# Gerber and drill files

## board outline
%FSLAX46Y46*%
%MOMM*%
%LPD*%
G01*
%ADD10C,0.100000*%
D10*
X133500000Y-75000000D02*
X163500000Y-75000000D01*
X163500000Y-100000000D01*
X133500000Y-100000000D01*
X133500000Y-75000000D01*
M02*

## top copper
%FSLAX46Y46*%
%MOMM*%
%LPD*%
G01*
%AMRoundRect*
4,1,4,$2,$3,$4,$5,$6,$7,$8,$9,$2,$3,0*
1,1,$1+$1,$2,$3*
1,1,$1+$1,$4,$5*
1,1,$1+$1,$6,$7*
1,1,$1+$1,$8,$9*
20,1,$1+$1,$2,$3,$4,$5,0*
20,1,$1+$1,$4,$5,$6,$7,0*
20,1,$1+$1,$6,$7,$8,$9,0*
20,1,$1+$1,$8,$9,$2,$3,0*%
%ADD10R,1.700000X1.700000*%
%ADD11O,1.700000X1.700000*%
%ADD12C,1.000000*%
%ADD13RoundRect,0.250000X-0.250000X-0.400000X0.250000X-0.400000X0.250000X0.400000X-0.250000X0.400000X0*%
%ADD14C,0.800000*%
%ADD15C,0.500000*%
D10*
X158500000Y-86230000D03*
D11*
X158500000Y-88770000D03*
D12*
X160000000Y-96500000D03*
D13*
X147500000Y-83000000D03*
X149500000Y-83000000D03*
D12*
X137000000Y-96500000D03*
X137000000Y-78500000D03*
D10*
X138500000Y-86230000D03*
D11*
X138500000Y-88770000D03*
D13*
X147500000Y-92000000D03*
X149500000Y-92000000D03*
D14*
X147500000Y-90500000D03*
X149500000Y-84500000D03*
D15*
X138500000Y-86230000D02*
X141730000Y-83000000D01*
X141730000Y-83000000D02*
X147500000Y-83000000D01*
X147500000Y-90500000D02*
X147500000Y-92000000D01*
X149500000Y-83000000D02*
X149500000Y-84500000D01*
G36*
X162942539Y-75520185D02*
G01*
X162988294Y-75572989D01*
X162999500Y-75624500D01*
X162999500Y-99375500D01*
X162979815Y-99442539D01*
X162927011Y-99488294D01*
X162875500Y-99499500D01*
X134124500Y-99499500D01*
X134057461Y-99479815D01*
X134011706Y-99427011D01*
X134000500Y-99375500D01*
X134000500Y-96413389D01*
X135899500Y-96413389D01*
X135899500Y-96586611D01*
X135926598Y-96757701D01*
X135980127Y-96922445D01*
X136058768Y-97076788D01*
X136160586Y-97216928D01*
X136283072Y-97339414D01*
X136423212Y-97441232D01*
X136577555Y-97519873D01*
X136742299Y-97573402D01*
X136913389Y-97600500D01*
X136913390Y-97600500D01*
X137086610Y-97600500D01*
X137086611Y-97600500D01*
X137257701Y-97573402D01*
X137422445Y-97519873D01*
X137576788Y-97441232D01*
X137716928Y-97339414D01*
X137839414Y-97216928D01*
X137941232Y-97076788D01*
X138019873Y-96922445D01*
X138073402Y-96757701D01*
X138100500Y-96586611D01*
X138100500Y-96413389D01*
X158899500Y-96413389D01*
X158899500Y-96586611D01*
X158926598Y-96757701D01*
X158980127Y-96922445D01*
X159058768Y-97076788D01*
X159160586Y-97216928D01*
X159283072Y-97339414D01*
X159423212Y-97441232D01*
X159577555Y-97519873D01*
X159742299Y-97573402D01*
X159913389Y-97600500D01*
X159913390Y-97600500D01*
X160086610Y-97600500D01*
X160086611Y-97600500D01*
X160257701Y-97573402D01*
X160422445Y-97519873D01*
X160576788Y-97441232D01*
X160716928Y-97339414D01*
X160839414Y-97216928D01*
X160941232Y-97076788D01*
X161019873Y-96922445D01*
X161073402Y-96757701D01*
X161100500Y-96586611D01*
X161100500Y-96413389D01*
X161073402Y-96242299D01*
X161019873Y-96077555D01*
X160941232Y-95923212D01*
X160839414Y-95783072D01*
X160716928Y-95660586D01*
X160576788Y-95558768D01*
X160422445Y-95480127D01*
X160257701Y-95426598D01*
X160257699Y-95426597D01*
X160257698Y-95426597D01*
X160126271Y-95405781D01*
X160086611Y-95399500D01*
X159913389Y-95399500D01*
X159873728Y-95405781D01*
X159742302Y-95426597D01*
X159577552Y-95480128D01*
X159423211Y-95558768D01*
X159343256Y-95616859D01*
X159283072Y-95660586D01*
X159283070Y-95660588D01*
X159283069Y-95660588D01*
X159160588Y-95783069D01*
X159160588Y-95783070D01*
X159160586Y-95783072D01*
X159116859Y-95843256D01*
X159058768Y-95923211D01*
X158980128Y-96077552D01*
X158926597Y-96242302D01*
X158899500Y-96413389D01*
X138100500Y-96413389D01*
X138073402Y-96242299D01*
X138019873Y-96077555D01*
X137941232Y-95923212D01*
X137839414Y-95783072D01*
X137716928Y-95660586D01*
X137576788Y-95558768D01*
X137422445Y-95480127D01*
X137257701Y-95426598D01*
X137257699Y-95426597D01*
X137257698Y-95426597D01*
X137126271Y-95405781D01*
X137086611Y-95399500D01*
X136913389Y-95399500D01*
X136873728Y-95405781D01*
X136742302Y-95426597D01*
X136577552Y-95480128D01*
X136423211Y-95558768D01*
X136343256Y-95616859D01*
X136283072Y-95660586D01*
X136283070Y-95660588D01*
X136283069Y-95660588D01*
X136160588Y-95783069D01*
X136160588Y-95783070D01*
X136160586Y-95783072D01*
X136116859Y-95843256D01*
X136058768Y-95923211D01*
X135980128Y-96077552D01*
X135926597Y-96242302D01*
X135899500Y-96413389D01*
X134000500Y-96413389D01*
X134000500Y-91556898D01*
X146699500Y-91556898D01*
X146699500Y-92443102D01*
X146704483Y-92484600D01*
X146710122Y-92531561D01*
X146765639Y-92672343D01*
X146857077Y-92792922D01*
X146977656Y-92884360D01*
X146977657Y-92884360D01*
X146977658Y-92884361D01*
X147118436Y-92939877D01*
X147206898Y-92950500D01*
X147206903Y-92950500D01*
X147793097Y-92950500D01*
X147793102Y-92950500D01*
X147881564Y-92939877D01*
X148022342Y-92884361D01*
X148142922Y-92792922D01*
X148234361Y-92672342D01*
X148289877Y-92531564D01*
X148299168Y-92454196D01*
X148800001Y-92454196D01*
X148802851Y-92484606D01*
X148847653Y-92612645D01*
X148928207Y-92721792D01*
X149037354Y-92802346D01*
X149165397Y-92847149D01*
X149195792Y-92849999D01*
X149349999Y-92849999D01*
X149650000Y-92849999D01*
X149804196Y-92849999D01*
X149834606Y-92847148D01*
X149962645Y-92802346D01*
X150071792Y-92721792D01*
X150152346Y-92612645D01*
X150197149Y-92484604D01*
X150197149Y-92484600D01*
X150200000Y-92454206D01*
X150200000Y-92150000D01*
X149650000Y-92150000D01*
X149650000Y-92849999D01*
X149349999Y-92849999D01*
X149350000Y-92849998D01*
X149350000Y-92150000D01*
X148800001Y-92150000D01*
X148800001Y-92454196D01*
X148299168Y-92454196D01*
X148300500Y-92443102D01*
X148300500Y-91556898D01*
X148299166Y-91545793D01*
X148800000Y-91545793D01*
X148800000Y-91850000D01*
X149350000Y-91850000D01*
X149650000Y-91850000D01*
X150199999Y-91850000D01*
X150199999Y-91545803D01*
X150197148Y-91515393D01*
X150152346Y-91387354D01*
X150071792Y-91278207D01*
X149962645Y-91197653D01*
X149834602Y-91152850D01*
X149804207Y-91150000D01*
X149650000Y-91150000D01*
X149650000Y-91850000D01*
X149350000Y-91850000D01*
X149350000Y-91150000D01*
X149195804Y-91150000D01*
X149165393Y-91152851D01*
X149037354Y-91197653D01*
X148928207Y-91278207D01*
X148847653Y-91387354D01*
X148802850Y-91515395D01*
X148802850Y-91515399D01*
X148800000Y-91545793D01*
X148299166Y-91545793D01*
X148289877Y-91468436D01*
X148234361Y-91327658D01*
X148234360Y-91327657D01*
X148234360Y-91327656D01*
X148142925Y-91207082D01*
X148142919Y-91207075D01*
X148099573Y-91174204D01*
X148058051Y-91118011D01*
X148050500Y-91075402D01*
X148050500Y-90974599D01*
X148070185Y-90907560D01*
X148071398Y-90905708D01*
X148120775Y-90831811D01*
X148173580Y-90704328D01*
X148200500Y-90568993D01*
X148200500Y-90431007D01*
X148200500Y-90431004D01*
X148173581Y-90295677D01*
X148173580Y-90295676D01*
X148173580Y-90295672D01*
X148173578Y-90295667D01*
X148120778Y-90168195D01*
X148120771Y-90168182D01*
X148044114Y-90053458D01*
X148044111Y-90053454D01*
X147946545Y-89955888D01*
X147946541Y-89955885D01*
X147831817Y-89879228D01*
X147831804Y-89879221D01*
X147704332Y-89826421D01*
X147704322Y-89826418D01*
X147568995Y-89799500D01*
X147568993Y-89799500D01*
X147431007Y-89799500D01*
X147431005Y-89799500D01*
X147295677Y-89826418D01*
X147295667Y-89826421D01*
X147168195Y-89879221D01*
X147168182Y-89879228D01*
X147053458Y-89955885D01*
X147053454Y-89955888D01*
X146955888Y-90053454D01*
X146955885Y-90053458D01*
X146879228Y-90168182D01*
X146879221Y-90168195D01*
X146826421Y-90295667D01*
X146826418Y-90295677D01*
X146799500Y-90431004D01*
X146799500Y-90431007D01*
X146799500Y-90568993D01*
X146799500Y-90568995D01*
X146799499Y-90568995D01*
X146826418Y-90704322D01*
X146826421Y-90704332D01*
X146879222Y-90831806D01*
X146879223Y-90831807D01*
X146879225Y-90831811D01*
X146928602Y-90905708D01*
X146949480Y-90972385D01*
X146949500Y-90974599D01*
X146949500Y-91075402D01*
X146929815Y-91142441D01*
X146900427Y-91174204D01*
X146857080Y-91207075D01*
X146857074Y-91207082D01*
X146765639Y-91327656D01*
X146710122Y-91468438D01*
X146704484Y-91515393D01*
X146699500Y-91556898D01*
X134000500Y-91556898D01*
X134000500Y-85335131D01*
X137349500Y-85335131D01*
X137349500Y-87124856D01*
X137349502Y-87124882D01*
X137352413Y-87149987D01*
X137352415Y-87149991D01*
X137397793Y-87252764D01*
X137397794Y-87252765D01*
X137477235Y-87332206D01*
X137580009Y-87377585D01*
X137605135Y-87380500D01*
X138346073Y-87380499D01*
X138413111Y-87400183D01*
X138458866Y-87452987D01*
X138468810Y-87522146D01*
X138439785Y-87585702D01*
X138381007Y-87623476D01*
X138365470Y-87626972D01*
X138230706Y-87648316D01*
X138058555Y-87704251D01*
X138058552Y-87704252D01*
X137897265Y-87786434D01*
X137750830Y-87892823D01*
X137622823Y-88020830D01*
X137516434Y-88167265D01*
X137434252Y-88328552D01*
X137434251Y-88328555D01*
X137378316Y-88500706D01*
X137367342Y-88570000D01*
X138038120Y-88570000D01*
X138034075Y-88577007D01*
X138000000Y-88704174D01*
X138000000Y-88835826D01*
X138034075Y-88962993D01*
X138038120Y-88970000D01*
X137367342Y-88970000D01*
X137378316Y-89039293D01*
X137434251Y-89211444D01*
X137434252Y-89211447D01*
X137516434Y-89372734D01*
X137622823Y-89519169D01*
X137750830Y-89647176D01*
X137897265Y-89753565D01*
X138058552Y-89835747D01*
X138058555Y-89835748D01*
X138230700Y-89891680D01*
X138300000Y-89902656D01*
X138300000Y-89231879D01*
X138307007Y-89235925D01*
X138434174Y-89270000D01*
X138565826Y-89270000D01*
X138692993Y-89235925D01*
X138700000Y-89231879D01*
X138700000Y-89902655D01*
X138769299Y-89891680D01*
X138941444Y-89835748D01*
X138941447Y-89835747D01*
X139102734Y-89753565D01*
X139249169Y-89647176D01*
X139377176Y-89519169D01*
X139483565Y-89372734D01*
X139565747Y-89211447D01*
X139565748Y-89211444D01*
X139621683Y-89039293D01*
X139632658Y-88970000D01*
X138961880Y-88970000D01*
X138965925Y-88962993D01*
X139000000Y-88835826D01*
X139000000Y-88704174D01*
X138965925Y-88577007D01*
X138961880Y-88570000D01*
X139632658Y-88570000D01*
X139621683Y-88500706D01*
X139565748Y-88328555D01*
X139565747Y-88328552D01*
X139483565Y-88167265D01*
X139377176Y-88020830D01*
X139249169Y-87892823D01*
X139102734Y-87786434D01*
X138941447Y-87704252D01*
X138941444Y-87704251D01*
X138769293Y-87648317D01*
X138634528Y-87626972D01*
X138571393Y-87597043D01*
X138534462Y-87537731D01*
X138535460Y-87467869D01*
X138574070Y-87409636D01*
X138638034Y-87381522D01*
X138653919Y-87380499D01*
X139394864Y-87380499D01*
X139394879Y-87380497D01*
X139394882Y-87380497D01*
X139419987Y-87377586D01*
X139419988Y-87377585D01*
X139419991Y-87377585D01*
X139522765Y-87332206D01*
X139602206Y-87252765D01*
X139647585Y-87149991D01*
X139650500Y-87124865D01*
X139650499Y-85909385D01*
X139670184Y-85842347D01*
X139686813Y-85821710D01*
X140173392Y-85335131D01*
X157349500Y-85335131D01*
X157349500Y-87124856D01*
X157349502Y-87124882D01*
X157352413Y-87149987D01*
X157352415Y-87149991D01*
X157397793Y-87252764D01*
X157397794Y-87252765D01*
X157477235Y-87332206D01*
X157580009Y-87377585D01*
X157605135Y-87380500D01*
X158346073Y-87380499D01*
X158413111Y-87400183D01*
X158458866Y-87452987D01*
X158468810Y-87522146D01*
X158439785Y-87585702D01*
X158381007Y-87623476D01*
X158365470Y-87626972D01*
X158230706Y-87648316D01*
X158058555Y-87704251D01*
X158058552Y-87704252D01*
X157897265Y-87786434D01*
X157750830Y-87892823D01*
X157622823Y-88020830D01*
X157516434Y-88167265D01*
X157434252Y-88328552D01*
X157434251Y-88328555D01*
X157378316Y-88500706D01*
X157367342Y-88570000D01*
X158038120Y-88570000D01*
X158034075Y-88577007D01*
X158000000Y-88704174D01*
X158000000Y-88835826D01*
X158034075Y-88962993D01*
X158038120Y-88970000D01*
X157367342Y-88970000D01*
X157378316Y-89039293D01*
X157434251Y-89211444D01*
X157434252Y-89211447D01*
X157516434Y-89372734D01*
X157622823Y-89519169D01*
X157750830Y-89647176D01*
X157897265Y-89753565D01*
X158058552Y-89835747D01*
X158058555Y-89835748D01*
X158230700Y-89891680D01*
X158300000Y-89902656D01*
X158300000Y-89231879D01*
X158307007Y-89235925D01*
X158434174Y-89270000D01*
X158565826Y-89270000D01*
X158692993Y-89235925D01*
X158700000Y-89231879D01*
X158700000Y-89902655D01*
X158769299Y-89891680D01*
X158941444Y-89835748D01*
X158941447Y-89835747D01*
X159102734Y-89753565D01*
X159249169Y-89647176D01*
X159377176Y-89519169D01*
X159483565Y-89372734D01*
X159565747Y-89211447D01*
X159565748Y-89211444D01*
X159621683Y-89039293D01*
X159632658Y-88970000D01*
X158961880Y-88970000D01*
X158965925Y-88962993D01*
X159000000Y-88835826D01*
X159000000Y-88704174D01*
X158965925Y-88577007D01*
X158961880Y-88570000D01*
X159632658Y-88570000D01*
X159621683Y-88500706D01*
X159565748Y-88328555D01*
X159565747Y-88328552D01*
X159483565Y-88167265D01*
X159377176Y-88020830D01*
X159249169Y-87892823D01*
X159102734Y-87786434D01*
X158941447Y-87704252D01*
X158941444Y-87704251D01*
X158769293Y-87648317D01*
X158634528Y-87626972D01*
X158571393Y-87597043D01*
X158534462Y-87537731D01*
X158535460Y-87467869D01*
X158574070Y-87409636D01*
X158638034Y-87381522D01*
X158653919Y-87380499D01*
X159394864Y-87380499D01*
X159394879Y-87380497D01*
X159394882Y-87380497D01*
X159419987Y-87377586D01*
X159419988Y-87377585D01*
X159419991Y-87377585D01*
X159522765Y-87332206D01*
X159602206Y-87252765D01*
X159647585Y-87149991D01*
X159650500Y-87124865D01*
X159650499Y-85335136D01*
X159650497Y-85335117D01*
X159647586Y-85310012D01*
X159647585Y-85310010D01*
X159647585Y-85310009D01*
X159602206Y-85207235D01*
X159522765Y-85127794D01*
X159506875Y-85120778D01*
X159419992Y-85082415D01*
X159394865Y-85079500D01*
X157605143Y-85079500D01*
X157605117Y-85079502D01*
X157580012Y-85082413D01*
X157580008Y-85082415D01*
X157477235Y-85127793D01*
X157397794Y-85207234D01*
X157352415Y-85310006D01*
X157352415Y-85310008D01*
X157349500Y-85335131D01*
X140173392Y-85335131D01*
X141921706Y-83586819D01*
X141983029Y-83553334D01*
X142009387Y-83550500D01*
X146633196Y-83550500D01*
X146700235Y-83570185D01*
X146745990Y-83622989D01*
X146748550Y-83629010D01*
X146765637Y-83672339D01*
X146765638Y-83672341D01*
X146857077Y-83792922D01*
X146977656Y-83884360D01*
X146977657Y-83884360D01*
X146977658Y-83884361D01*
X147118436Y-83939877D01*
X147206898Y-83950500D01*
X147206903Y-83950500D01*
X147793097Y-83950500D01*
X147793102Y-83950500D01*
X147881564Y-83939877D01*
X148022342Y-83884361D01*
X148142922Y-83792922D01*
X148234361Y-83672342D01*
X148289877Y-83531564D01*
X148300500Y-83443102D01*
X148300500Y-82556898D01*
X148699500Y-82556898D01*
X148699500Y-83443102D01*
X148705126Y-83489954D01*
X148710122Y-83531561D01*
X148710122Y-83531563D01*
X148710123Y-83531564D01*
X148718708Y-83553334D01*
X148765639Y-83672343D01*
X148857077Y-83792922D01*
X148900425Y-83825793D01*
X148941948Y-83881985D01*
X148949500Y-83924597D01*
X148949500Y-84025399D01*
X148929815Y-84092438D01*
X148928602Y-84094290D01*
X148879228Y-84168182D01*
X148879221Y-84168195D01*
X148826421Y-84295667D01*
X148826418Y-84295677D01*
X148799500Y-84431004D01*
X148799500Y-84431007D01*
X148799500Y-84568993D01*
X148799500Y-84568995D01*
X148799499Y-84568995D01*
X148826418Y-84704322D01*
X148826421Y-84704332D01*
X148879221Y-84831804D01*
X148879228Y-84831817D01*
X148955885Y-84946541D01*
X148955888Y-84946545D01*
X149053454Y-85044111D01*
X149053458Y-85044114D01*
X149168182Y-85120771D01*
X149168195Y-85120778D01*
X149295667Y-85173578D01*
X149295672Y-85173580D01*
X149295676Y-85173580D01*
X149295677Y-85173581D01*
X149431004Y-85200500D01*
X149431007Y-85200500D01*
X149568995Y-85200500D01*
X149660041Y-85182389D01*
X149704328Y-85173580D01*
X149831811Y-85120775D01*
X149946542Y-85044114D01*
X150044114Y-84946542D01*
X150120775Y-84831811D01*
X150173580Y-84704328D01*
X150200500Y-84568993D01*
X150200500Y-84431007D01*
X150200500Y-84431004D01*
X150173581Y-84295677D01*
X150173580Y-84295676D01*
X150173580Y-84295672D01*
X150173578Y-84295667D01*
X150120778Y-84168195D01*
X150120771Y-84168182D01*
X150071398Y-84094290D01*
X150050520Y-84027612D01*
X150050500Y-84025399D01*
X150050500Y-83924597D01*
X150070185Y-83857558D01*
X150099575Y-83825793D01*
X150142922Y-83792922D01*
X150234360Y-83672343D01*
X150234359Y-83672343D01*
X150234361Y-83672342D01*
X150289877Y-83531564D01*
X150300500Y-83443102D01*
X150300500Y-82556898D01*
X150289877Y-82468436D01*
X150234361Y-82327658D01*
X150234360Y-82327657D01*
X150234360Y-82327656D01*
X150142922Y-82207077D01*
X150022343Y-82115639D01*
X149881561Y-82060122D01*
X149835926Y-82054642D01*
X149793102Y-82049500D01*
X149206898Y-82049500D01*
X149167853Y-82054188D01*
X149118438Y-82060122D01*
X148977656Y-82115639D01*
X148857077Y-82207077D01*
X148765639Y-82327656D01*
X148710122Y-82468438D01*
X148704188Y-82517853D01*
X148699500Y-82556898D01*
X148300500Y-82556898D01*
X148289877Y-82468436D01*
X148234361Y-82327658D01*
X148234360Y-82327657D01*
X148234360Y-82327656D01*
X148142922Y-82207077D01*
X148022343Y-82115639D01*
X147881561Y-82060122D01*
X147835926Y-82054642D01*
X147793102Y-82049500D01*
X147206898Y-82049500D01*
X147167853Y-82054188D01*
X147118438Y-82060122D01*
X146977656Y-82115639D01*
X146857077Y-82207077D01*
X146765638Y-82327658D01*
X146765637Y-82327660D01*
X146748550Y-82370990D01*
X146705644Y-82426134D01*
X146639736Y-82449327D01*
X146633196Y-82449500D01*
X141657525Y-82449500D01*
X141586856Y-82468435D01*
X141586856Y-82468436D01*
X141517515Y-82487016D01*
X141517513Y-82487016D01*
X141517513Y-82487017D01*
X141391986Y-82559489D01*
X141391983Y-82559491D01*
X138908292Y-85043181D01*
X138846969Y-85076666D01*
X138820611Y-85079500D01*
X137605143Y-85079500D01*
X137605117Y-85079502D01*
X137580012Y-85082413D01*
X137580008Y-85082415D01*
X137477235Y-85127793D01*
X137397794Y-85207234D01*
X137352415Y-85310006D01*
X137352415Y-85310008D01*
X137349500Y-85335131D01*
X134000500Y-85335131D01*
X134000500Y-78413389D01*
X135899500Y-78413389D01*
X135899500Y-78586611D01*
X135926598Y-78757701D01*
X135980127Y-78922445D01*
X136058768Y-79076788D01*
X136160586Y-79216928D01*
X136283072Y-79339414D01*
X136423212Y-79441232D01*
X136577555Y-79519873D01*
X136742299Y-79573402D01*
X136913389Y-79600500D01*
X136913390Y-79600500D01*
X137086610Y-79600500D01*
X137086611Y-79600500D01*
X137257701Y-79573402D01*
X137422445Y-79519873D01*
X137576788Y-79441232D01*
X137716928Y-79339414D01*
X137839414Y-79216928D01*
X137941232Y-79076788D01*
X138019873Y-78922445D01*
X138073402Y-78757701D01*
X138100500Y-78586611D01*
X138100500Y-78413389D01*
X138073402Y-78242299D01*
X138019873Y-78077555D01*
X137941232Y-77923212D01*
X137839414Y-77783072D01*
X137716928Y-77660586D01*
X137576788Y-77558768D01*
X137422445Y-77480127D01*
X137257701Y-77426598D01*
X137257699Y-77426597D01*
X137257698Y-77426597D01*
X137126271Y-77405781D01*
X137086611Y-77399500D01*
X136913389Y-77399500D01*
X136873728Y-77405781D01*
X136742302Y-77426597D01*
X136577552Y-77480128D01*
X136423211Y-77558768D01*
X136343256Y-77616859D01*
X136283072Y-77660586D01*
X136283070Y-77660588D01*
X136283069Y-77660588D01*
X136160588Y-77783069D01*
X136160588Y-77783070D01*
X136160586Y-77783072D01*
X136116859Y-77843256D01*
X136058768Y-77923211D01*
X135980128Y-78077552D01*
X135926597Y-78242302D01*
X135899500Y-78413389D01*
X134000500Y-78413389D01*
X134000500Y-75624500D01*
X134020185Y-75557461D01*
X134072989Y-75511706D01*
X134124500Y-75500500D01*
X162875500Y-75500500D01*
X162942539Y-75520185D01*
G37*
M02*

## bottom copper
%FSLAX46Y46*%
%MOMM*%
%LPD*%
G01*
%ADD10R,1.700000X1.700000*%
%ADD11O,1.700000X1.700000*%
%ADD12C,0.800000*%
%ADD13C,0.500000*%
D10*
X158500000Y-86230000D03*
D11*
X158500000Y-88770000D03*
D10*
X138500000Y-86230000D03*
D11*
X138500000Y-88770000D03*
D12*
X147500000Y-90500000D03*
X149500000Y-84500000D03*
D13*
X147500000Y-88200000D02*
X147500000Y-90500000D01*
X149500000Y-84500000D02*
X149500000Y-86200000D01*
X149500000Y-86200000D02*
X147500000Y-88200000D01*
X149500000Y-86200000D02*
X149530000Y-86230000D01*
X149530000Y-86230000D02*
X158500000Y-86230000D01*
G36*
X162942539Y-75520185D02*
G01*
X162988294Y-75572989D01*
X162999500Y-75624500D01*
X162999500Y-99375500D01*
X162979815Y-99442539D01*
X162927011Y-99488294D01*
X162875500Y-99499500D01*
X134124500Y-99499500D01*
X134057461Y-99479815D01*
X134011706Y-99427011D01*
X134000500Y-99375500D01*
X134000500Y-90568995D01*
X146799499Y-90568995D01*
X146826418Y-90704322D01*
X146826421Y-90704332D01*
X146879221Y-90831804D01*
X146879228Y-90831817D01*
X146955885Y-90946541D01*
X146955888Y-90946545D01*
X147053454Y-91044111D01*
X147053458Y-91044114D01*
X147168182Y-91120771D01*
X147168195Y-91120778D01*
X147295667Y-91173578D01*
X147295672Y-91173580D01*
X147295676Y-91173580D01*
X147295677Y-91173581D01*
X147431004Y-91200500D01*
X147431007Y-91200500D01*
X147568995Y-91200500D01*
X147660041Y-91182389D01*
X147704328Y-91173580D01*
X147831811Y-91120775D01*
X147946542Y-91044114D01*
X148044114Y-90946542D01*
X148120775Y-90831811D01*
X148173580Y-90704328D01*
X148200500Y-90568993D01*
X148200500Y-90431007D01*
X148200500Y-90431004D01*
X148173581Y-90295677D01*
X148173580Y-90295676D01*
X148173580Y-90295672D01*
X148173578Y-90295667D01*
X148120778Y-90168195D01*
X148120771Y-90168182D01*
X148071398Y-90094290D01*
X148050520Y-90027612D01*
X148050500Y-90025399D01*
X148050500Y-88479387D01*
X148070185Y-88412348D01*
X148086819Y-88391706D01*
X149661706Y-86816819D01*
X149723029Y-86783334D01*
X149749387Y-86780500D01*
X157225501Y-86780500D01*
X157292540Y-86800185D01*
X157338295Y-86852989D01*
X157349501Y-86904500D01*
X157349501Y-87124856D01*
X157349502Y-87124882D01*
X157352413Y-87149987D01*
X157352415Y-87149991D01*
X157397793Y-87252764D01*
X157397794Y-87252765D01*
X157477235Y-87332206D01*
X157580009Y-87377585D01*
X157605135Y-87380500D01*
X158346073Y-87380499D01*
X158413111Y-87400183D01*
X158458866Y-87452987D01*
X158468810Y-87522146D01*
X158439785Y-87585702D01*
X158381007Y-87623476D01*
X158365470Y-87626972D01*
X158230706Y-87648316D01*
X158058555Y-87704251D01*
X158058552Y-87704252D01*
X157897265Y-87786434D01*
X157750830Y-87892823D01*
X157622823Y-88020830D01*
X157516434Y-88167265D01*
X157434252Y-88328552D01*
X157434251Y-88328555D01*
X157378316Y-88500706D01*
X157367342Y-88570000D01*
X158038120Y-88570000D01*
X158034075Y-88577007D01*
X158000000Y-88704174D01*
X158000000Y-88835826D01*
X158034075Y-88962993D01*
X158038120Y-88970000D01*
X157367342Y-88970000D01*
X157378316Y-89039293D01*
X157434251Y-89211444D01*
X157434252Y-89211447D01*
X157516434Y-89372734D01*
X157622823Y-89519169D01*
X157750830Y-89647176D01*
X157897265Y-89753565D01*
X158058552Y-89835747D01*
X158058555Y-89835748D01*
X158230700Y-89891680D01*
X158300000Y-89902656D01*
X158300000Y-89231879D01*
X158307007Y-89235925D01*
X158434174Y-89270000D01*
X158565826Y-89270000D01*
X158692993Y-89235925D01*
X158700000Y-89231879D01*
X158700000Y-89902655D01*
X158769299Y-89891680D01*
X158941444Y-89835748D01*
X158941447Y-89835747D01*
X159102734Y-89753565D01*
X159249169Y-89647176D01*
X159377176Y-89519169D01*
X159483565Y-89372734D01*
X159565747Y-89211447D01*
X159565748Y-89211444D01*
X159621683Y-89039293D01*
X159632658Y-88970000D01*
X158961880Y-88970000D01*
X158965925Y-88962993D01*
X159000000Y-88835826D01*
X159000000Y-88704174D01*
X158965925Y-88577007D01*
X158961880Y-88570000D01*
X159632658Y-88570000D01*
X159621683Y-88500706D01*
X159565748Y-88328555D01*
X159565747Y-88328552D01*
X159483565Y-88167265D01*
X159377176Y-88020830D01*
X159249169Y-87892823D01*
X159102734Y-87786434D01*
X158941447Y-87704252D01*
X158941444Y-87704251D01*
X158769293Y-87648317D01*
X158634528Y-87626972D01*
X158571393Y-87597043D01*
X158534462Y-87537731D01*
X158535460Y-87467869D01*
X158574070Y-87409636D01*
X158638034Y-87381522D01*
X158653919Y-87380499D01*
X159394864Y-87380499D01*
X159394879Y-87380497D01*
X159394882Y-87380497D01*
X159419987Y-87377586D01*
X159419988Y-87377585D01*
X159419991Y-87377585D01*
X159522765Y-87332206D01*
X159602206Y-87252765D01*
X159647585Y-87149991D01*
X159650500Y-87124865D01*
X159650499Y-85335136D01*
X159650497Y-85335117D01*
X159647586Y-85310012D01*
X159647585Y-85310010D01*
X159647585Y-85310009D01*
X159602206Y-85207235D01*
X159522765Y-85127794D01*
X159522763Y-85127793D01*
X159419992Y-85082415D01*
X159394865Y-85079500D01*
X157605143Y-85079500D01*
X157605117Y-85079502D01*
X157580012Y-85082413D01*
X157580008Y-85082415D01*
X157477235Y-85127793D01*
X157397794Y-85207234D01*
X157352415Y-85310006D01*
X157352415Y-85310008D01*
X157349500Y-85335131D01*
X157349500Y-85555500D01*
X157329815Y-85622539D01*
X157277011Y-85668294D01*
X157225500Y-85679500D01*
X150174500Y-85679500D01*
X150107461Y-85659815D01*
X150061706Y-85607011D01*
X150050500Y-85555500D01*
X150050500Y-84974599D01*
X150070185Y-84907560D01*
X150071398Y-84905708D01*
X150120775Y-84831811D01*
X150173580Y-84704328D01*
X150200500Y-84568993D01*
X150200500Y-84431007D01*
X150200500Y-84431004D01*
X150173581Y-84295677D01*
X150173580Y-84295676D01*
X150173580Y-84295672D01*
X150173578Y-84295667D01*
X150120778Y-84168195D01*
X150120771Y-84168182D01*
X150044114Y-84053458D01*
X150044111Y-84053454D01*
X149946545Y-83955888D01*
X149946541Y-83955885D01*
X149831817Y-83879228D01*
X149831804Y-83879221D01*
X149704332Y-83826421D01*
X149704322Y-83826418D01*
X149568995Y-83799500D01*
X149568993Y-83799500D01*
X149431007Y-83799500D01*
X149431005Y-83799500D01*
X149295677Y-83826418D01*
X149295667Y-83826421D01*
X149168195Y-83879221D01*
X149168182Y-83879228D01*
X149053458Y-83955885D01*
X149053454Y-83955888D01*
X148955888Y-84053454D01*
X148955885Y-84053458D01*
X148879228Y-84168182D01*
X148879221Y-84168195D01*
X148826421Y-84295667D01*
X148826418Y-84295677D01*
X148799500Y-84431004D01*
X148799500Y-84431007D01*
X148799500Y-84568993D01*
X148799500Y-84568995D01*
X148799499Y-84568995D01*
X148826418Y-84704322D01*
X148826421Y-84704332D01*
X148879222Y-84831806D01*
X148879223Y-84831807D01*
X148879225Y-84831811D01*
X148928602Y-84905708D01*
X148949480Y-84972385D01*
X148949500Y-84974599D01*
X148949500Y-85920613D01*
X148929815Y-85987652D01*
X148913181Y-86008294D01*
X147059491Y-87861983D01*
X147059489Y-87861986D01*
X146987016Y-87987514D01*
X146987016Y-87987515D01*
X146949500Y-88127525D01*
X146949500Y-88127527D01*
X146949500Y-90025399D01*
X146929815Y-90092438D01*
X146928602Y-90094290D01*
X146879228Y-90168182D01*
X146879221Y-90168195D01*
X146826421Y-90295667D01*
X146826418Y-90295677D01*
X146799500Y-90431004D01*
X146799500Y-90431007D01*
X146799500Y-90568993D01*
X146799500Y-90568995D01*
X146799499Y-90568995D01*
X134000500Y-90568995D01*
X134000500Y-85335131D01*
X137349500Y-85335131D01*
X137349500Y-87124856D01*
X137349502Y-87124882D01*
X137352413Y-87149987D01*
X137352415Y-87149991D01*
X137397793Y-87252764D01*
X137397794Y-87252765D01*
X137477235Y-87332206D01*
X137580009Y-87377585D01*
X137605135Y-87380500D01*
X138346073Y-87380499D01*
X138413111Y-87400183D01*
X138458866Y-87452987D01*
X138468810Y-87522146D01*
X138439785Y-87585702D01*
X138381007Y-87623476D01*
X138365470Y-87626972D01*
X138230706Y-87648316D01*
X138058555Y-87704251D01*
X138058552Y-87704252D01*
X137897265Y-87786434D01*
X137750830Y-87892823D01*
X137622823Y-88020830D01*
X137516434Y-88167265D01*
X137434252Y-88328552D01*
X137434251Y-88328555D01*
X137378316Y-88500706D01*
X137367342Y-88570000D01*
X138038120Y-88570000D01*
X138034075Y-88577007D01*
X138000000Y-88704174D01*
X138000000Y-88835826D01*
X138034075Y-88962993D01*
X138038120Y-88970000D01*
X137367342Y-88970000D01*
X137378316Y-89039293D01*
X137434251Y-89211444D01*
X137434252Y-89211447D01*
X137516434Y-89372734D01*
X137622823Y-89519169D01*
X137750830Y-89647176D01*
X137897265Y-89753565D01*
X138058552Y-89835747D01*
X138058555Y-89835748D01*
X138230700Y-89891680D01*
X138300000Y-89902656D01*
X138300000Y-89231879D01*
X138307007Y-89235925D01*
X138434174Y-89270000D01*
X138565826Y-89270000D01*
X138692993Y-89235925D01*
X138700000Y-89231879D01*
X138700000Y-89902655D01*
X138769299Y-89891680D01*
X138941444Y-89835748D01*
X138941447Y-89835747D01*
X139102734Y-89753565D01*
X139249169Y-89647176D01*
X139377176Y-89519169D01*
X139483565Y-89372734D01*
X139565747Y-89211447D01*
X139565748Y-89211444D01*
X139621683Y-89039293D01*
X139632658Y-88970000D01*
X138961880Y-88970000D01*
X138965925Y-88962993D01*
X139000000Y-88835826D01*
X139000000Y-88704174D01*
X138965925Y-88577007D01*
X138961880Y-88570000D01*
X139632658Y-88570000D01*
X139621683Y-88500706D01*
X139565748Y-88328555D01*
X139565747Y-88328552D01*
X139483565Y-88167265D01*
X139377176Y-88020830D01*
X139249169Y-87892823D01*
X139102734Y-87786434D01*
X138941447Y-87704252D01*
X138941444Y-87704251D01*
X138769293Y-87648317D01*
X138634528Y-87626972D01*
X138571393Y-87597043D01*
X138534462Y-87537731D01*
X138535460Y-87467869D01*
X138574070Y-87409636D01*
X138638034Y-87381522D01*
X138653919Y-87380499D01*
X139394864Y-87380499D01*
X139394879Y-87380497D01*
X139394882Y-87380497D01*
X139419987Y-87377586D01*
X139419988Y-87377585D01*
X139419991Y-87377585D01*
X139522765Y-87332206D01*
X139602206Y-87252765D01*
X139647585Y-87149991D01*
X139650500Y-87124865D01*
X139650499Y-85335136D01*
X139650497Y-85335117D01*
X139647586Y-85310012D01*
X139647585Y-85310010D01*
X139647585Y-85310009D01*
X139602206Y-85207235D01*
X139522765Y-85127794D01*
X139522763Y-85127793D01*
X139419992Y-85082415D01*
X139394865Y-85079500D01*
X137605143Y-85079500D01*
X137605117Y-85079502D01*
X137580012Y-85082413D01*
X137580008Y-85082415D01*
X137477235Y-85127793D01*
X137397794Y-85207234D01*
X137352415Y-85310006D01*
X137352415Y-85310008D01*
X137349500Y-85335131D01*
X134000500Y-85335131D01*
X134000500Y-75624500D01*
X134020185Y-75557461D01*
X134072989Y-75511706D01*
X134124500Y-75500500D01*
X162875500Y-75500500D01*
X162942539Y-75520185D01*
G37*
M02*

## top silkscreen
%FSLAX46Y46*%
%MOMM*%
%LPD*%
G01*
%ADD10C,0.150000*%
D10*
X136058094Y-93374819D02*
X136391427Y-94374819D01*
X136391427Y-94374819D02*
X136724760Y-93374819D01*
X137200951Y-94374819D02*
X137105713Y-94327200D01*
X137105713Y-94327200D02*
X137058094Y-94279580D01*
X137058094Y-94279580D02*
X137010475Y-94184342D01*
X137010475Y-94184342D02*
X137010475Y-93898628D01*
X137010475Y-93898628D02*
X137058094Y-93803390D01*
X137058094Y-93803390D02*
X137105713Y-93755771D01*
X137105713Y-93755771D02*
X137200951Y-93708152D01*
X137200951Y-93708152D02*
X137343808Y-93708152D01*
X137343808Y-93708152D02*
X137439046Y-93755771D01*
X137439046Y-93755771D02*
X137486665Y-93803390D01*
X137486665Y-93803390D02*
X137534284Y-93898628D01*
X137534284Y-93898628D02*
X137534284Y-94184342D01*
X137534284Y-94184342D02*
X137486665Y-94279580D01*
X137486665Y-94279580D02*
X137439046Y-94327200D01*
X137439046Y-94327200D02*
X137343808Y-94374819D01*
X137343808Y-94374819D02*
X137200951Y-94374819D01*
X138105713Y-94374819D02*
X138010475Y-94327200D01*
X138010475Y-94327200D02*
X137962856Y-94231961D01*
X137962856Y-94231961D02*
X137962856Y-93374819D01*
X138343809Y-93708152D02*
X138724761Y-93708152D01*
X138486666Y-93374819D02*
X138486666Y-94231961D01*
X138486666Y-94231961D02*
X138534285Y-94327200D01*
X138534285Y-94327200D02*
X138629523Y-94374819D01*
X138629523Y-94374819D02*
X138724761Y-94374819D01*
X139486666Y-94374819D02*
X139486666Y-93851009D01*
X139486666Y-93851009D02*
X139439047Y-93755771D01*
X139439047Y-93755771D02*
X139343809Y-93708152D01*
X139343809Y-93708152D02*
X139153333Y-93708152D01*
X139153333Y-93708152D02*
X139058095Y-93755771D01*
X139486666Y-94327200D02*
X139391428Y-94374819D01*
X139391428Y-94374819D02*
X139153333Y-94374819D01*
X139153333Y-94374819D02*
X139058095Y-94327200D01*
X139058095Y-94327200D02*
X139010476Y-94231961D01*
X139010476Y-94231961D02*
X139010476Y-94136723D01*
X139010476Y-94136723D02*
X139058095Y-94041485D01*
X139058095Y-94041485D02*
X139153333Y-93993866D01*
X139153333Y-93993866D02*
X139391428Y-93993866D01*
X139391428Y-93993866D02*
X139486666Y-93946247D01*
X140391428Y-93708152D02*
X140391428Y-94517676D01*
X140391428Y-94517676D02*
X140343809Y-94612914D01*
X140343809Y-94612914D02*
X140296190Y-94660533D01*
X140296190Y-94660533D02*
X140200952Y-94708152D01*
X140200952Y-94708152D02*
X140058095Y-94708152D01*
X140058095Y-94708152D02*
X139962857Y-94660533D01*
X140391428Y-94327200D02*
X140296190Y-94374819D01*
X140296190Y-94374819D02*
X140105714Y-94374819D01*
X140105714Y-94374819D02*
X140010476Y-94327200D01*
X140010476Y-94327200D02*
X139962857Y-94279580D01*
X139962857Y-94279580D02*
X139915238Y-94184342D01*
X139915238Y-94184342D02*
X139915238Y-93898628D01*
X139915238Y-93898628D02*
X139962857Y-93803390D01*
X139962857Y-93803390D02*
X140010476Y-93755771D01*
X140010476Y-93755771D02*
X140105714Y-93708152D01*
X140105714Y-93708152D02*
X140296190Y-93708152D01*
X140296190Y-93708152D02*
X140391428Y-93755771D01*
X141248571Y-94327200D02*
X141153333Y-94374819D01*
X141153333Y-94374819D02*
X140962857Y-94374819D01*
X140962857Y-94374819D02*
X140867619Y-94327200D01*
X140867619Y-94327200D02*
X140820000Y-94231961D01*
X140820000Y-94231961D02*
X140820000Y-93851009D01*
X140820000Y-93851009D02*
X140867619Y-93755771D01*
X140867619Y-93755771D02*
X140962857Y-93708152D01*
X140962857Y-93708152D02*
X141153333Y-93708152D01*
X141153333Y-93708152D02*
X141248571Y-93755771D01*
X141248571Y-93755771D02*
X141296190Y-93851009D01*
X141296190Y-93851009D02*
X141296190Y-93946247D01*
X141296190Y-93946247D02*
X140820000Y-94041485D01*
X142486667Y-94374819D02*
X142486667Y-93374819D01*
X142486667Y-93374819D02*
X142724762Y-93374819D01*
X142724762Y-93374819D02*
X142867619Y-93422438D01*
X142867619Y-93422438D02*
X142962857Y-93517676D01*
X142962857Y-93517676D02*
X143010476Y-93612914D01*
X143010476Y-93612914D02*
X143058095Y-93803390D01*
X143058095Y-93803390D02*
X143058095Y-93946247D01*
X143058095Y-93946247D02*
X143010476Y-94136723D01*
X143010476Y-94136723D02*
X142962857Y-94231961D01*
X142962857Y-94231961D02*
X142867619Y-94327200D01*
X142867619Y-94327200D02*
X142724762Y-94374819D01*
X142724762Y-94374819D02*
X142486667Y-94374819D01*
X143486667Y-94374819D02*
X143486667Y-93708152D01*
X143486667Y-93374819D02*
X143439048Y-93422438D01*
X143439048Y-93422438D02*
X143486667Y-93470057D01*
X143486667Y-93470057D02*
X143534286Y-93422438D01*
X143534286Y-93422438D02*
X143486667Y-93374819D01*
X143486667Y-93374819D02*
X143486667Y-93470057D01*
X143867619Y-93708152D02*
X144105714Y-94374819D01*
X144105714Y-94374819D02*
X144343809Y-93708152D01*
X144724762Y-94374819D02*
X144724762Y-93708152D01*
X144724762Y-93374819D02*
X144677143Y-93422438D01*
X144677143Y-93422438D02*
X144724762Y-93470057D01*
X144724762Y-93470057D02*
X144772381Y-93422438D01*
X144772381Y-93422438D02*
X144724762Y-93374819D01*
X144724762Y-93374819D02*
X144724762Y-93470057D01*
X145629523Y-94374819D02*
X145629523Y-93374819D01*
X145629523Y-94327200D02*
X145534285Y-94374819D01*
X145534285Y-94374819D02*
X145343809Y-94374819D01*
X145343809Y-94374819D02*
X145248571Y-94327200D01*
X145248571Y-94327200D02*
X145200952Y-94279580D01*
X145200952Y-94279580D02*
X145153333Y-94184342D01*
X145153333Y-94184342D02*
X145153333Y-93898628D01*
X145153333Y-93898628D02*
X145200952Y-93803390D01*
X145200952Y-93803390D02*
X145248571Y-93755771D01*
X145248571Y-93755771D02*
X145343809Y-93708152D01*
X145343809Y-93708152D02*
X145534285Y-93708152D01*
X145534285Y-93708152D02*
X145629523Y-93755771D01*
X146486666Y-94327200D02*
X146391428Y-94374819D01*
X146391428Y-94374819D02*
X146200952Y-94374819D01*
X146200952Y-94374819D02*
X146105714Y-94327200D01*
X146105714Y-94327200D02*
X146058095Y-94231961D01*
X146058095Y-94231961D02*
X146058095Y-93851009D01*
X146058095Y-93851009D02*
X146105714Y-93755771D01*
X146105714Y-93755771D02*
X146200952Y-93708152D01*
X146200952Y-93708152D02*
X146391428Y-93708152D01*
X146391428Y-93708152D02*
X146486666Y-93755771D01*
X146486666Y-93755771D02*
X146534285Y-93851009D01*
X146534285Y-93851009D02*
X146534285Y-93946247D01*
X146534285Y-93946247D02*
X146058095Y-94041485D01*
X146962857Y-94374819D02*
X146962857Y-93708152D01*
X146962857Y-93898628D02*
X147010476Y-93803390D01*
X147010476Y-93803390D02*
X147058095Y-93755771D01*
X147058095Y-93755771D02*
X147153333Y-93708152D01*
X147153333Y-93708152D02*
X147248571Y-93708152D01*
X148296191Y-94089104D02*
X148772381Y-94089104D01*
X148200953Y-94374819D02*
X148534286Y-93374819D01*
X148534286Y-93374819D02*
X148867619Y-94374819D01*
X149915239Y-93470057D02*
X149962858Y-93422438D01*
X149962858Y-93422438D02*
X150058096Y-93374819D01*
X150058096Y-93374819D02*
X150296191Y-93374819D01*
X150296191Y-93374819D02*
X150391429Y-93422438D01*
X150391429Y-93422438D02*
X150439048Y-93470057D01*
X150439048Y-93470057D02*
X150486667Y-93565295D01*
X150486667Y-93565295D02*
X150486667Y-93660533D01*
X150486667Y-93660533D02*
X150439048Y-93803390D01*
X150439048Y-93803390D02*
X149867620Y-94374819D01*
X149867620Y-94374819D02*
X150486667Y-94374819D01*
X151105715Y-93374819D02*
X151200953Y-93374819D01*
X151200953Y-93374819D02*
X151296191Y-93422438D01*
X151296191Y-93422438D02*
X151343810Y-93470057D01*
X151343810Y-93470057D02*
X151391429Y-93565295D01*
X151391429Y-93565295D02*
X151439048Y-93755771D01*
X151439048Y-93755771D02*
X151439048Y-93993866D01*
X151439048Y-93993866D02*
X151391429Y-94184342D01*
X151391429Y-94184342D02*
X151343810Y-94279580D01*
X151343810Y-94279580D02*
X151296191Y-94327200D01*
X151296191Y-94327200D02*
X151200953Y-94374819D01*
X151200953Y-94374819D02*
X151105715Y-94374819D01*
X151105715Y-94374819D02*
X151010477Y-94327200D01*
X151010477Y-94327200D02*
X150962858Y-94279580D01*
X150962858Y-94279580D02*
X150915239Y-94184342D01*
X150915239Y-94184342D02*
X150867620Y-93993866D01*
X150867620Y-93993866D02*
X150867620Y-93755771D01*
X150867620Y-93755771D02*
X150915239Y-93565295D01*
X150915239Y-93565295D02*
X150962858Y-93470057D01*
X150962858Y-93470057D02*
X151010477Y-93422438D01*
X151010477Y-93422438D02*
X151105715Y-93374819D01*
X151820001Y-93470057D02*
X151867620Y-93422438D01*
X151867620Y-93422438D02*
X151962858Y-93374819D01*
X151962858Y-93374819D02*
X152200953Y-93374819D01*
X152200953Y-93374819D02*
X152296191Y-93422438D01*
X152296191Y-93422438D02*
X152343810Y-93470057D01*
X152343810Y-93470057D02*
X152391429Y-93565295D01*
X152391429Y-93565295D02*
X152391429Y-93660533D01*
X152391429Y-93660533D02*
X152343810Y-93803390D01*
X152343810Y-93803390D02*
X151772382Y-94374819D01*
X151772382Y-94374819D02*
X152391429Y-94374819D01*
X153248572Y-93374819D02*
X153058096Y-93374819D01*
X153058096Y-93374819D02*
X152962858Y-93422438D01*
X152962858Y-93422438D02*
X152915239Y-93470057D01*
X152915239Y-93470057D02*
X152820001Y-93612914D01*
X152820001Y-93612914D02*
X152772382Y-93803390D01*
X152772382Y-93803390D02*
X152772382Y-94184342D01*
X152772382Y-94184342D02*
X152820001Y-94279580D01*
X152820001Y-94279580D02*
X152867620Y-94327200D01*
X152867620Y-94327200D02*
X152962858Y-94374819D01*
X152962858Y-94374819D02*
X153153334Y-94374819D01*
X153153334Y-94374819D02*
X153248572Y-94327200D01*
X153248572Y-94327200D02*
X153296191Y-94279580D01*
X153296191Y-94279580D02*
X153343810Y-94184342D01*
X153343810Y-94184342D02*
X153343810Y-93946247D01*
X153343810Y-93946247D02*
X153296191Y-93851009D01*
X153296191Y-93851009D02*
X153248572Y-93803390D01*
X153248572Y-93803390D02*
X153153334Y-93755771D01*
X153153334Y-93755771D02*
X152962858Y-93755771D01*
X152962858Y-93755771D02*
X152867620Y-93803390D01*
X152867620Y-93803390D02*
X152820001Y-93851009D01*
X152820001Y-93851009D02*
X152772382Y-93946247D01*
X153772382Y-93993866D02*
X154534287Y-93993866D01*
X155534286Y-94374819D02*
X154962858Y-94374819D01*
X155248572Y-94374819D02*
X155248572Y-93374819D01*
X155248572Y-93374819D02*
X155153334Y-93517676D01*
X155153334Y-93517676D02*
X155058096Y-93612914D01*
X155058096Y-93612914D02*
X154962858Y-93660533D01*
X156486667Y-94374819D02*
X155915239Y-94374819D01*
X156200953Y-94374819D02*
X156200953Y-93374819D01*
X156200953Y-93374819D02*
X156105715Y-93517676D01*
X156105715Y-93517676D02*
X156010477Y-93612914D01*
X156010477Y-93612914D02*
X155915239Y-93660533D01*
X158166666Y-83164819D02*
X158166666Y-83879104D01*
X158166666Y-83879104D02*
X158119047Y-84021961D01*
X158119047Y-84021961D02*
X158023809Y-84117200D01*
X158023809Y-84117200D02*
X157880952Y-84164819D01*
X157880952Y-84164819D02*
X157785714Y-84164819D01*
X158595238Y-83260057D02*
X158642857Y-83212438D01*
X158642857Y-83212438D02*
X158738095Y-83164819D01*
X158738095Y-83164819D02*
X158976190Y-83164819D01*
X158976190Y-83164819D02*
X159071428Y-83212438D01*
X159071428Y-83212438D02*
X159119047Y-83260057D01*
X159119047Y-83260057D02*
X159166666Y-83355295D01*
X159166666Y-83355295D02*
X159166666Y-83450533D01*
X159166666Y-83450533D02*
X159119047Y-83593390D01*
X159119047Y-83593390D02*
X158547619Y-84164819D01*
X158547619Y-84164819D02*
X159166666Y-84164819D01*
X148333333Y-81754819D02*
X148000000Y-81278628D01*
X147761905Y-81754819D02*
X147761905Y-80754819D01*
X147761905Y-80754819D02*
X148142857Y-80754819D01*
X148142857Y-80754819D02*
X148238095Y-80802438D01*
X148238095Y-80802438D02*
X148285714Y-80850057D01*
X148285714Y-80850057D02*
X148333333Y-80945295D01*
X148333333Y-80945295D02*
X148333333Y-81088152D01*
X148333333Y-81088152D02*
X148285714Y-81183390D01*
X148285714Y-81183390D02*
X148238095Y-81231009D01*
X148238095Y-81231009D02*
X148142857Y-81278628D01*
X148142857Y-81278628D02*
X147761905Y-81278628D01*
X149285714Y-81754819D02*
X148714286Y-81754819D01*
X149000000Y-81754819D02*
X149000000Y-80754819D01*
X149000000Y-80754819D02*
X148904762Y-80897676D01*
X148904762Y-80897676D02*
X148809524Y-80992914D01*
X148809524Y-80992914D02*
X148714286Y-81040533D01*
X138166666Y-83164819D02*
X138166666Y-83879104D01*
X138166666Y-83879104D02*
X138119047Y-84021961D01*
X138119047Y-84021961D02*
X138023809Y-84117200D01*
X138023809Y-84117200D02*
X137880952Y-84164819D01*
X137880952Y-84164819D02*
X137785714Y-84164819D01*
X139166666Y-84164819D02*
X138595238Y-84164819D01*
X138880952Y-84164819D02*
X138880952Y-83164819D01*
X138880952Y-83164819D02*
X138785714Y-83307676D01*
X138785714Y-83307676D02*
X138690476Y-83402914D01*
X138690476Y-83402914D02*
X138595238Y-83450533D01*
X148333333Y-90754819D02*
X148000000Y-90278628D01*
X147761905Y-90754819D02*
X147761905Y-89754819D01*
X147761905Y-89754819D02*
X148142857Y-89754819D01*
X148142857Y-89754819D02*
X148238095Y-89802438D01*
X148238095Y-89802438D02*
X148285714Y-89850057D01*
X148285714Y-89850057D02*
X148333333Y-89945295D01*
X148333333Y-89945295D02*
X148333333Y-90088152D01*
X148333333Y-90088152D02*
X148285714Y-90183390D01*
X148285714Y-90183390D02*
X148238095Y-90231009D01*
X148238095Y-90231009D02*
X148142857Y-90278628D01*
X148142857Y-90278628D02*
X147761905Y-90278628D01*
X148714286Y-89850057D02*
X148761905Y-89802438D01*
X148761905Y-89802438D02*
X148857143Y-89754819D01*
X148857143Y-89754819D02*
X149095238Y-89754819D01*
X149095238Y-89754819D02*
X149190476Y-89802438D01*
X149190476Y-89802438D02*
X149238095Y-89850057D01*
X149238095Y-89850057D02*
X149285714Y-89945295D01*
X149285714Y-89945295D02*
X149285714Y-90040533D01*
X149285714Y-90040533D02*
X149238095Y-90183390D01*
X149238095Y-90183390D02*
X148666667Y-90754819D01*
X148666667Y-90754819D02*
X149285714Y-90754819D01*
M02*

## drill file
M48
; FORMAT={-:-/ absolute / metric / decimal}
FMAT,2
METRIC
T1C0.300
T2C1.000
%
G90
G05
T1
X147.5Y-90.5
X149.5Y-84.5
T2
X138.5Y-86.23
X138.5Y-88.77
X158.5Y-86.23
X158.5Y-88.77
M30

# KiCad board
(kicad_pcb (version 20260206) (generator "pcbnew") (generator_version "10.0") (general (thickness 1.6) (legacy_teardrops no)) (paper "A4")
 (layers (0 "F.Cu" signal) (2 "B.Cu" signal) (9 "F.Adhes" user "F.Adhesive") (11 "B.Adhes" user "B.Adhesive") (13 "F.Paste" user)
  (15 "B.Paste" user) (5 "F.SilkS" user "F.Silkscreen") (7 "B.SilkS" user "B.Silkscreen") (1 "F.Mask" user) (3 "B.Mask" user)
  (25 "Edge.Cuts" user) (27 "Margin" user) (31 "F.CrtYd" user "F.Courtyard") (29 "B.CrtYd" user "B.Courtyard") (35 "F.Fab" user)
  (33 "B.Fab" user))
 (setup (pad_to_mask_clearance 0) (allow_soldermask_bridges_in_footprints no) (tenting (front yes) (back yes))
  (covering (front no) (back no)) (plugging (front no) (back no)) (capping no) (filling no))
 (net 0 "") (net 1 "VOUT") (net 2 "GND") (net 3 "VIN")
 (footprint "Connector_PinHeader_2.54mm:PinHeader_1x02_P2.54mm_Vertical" (layer "F.Cu") (at 158.5 87.5)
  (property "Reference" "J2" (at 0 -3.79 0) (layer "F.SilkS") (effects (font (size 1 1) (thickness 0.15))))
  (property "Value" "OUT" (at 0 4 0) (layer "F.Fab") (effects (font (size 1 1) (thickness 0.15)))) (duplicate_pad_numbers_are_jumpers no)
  (pad "1" thru_hole rect (at 0 -1.27) (size 1.7 1.7) (drill 1) (layers "*.Cu" "*.Mask") (remove_unused_layers no) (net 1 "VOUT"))
  (pad "2" thru_hole oval (at 0 1.27) (size 1.7 1.7) (drill 1) (layers "*.Cu" "*.Mask") (remove_unused_layers no) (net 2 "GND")))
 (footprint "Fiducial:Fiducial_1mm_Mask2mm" (layer "F.Cu") (at 160 96.5)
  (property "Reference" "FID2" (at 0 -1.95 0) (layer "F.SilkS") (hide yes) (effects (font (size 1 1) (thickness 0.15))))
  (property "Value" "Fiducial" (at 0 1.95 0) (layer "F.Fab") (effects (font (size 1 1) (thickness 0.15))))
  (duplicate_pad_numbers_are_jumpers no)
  (pad "" smd circle (at 0 0) (size 1 1) (layers "F.Cu" "F.Mask") (solder_mask_margin 0.5) (clearance 0.6)))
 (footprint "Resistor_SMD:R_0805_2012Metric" (layer "F.Cu") (at 148.5 83)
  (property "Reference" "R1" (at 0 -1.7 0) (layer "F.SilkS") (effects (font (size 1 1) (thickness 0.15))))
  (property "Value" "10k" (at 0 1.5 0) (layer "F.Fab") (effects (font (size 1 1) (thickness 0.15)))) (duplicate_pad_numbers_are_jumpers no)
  (pad "1" smd roundrect (at -1 0) (size 1 1.3) (layers "F.Cu" "F.Mask" "F.Paste") (roundrect_rratio 0.25) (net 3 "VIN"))
  (pad "2" smd roundrect (at 1 0) (size 1 1.3) (layers "F.Cu" "F.Mask" "F.Paste") (roundrect_rratio 0.25) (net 1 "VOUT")))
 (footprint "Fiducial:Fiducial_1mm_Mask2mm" (layer "F.Cu") (at 137 96.5)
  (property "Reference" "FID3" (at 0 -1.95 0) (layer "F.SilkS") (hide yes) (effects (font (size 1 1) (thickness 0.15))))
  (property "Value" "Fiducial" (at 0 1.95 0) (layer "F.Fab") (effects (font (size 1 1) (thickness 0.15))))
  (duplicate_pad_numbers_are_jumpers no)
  (pad "" smd circle (at 0 0) (size 1 1) (layers "F.Cu" "F.Mask") (solder_mask_margin 0.5) (clearance 0.6)))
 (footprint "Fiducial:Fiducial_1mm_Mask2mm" (layer "F.Cu") (at 137 78.5)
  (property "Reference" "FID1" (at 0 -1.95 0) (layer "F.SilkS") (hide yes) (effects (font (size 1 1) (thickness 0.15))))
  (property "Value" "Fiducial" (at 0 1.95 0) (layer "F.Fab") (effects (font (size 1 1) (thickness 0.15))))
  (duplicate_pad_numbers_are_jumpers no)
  (pad "" smd circle (at 0 0) (size 1 1) (layers "F.Cu" "F.Mask") (solder_mask_margin 0.5) (clearance 0.6)))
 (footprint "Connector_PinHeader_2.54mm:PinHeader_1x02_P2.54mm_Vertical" (layer "F.Cu") (at 138.5 87.5)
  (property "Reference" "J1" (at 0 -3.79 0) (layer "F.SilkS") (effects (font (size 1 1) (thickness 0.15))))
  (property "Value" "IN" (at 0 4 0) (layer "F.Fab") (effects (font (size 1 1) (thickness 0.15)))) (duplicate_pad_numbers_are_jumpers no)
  (pad "1" thru_hole rect (at 0 -1.27) (size 1.7 1.7) (drill 1) (layers "*.Cu" "*.Mask") (remove_unused_layers no) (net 3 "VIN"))
  (pad "2" thru_hole oval (at 0 1.27) (size 1.7 1.7) (drill 1) (layers "*.Cu" "*.Mask") (remove_unused_layers no) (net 2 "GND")))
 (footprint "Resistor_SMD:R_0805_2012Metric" (layer "F.Cu") (at 148.5 92)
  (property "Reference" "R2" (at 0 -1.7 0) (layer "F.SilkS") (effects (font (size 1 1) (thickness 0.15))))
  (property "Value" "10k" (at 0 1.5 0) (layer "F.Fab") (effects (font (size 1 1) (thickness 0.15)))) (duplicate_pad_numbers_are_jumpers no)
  (pad "1" smd roundrect (at -1 0) (size 1 1.3) (layers "F.Cu" "F.Mask" "F.Paste") (roundrect_rratio 0.25) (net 1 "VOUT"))
  (pad "2" smd roundrect (at 1 0) (size 1 1.3) (layers "F.Cu" "F.Mask" "F.Paste") (roundrect_rratio 0.25) (thermal_bridge_width 0.3)
   (thermal_gap 0.2) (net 2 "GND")))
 (gr_rect (start 133.5 75) (end 163.5 100) (stroke (width 0.1) (type default)) (fill no) (layer "Edge.Cuts"))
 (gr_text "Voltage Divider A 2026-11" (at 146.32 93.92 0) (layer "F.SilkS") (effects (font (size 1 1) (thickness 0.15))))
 (segment (start 138.5 86.23) (end 141.73 83) (width 0.5) (layer "F.Cu") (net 3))
 (segment (start 141.73 83) (end 147.5 83) (width 0.5) (layer "F.Cu") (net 3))
 (segment (start 147.5 90.5) (end 147.5 92) (width 0.5) (layer "F.Cu") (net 1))
 (segment (start 149.5 83) (end 149.5 84.5) (width 0.5) (layer "F.Cu") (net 1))
 (via (at 147.5 90.5) (size 0.8) (drill 0.3) (layers "F.Cu" "B.Cu") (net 1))
 (via (at 149.5 84.5) (size 0.8) (drill 0.3) (layers "F.Cu" "B.Cu") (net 1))
 (segment (start 147.5 88.2) (end 147.5 90.5) (width 0.5) (layer "B.Cu") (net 1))
 (segment (start 149.5 84.5) (end 149.5 86.2) (width 0.5) (layer "B.Cu") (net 1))
 (segment (start 149.5 86.2) (end 147.5 88.2) (width 0.5) (layer "B.Cu") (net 1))
 (segment (start 149.5 86.2) (end 149.53 86.23) (width 0.5) (layer "B.Cu") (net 1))
 (segment (start 149.53 86.23) (end 158.5 86.23) (width 0.5) (layer "B.Cu") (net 1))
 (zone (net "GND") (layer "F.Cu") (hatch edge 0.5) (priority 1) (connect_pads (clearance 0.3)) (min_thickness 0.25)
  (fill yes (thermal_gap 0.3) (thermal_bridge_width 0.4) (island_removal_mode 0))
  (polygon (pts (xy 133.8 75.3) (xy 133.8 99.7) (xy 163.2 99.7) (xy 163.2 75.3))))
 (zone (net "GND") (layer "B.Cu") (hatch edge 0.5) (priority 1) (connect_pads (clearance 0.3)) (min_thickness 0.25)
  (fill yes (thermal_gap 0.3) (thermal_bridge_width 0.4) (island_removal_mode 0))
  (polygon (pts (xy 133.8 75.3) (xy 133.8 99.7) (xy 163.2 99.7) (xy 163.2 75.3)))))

